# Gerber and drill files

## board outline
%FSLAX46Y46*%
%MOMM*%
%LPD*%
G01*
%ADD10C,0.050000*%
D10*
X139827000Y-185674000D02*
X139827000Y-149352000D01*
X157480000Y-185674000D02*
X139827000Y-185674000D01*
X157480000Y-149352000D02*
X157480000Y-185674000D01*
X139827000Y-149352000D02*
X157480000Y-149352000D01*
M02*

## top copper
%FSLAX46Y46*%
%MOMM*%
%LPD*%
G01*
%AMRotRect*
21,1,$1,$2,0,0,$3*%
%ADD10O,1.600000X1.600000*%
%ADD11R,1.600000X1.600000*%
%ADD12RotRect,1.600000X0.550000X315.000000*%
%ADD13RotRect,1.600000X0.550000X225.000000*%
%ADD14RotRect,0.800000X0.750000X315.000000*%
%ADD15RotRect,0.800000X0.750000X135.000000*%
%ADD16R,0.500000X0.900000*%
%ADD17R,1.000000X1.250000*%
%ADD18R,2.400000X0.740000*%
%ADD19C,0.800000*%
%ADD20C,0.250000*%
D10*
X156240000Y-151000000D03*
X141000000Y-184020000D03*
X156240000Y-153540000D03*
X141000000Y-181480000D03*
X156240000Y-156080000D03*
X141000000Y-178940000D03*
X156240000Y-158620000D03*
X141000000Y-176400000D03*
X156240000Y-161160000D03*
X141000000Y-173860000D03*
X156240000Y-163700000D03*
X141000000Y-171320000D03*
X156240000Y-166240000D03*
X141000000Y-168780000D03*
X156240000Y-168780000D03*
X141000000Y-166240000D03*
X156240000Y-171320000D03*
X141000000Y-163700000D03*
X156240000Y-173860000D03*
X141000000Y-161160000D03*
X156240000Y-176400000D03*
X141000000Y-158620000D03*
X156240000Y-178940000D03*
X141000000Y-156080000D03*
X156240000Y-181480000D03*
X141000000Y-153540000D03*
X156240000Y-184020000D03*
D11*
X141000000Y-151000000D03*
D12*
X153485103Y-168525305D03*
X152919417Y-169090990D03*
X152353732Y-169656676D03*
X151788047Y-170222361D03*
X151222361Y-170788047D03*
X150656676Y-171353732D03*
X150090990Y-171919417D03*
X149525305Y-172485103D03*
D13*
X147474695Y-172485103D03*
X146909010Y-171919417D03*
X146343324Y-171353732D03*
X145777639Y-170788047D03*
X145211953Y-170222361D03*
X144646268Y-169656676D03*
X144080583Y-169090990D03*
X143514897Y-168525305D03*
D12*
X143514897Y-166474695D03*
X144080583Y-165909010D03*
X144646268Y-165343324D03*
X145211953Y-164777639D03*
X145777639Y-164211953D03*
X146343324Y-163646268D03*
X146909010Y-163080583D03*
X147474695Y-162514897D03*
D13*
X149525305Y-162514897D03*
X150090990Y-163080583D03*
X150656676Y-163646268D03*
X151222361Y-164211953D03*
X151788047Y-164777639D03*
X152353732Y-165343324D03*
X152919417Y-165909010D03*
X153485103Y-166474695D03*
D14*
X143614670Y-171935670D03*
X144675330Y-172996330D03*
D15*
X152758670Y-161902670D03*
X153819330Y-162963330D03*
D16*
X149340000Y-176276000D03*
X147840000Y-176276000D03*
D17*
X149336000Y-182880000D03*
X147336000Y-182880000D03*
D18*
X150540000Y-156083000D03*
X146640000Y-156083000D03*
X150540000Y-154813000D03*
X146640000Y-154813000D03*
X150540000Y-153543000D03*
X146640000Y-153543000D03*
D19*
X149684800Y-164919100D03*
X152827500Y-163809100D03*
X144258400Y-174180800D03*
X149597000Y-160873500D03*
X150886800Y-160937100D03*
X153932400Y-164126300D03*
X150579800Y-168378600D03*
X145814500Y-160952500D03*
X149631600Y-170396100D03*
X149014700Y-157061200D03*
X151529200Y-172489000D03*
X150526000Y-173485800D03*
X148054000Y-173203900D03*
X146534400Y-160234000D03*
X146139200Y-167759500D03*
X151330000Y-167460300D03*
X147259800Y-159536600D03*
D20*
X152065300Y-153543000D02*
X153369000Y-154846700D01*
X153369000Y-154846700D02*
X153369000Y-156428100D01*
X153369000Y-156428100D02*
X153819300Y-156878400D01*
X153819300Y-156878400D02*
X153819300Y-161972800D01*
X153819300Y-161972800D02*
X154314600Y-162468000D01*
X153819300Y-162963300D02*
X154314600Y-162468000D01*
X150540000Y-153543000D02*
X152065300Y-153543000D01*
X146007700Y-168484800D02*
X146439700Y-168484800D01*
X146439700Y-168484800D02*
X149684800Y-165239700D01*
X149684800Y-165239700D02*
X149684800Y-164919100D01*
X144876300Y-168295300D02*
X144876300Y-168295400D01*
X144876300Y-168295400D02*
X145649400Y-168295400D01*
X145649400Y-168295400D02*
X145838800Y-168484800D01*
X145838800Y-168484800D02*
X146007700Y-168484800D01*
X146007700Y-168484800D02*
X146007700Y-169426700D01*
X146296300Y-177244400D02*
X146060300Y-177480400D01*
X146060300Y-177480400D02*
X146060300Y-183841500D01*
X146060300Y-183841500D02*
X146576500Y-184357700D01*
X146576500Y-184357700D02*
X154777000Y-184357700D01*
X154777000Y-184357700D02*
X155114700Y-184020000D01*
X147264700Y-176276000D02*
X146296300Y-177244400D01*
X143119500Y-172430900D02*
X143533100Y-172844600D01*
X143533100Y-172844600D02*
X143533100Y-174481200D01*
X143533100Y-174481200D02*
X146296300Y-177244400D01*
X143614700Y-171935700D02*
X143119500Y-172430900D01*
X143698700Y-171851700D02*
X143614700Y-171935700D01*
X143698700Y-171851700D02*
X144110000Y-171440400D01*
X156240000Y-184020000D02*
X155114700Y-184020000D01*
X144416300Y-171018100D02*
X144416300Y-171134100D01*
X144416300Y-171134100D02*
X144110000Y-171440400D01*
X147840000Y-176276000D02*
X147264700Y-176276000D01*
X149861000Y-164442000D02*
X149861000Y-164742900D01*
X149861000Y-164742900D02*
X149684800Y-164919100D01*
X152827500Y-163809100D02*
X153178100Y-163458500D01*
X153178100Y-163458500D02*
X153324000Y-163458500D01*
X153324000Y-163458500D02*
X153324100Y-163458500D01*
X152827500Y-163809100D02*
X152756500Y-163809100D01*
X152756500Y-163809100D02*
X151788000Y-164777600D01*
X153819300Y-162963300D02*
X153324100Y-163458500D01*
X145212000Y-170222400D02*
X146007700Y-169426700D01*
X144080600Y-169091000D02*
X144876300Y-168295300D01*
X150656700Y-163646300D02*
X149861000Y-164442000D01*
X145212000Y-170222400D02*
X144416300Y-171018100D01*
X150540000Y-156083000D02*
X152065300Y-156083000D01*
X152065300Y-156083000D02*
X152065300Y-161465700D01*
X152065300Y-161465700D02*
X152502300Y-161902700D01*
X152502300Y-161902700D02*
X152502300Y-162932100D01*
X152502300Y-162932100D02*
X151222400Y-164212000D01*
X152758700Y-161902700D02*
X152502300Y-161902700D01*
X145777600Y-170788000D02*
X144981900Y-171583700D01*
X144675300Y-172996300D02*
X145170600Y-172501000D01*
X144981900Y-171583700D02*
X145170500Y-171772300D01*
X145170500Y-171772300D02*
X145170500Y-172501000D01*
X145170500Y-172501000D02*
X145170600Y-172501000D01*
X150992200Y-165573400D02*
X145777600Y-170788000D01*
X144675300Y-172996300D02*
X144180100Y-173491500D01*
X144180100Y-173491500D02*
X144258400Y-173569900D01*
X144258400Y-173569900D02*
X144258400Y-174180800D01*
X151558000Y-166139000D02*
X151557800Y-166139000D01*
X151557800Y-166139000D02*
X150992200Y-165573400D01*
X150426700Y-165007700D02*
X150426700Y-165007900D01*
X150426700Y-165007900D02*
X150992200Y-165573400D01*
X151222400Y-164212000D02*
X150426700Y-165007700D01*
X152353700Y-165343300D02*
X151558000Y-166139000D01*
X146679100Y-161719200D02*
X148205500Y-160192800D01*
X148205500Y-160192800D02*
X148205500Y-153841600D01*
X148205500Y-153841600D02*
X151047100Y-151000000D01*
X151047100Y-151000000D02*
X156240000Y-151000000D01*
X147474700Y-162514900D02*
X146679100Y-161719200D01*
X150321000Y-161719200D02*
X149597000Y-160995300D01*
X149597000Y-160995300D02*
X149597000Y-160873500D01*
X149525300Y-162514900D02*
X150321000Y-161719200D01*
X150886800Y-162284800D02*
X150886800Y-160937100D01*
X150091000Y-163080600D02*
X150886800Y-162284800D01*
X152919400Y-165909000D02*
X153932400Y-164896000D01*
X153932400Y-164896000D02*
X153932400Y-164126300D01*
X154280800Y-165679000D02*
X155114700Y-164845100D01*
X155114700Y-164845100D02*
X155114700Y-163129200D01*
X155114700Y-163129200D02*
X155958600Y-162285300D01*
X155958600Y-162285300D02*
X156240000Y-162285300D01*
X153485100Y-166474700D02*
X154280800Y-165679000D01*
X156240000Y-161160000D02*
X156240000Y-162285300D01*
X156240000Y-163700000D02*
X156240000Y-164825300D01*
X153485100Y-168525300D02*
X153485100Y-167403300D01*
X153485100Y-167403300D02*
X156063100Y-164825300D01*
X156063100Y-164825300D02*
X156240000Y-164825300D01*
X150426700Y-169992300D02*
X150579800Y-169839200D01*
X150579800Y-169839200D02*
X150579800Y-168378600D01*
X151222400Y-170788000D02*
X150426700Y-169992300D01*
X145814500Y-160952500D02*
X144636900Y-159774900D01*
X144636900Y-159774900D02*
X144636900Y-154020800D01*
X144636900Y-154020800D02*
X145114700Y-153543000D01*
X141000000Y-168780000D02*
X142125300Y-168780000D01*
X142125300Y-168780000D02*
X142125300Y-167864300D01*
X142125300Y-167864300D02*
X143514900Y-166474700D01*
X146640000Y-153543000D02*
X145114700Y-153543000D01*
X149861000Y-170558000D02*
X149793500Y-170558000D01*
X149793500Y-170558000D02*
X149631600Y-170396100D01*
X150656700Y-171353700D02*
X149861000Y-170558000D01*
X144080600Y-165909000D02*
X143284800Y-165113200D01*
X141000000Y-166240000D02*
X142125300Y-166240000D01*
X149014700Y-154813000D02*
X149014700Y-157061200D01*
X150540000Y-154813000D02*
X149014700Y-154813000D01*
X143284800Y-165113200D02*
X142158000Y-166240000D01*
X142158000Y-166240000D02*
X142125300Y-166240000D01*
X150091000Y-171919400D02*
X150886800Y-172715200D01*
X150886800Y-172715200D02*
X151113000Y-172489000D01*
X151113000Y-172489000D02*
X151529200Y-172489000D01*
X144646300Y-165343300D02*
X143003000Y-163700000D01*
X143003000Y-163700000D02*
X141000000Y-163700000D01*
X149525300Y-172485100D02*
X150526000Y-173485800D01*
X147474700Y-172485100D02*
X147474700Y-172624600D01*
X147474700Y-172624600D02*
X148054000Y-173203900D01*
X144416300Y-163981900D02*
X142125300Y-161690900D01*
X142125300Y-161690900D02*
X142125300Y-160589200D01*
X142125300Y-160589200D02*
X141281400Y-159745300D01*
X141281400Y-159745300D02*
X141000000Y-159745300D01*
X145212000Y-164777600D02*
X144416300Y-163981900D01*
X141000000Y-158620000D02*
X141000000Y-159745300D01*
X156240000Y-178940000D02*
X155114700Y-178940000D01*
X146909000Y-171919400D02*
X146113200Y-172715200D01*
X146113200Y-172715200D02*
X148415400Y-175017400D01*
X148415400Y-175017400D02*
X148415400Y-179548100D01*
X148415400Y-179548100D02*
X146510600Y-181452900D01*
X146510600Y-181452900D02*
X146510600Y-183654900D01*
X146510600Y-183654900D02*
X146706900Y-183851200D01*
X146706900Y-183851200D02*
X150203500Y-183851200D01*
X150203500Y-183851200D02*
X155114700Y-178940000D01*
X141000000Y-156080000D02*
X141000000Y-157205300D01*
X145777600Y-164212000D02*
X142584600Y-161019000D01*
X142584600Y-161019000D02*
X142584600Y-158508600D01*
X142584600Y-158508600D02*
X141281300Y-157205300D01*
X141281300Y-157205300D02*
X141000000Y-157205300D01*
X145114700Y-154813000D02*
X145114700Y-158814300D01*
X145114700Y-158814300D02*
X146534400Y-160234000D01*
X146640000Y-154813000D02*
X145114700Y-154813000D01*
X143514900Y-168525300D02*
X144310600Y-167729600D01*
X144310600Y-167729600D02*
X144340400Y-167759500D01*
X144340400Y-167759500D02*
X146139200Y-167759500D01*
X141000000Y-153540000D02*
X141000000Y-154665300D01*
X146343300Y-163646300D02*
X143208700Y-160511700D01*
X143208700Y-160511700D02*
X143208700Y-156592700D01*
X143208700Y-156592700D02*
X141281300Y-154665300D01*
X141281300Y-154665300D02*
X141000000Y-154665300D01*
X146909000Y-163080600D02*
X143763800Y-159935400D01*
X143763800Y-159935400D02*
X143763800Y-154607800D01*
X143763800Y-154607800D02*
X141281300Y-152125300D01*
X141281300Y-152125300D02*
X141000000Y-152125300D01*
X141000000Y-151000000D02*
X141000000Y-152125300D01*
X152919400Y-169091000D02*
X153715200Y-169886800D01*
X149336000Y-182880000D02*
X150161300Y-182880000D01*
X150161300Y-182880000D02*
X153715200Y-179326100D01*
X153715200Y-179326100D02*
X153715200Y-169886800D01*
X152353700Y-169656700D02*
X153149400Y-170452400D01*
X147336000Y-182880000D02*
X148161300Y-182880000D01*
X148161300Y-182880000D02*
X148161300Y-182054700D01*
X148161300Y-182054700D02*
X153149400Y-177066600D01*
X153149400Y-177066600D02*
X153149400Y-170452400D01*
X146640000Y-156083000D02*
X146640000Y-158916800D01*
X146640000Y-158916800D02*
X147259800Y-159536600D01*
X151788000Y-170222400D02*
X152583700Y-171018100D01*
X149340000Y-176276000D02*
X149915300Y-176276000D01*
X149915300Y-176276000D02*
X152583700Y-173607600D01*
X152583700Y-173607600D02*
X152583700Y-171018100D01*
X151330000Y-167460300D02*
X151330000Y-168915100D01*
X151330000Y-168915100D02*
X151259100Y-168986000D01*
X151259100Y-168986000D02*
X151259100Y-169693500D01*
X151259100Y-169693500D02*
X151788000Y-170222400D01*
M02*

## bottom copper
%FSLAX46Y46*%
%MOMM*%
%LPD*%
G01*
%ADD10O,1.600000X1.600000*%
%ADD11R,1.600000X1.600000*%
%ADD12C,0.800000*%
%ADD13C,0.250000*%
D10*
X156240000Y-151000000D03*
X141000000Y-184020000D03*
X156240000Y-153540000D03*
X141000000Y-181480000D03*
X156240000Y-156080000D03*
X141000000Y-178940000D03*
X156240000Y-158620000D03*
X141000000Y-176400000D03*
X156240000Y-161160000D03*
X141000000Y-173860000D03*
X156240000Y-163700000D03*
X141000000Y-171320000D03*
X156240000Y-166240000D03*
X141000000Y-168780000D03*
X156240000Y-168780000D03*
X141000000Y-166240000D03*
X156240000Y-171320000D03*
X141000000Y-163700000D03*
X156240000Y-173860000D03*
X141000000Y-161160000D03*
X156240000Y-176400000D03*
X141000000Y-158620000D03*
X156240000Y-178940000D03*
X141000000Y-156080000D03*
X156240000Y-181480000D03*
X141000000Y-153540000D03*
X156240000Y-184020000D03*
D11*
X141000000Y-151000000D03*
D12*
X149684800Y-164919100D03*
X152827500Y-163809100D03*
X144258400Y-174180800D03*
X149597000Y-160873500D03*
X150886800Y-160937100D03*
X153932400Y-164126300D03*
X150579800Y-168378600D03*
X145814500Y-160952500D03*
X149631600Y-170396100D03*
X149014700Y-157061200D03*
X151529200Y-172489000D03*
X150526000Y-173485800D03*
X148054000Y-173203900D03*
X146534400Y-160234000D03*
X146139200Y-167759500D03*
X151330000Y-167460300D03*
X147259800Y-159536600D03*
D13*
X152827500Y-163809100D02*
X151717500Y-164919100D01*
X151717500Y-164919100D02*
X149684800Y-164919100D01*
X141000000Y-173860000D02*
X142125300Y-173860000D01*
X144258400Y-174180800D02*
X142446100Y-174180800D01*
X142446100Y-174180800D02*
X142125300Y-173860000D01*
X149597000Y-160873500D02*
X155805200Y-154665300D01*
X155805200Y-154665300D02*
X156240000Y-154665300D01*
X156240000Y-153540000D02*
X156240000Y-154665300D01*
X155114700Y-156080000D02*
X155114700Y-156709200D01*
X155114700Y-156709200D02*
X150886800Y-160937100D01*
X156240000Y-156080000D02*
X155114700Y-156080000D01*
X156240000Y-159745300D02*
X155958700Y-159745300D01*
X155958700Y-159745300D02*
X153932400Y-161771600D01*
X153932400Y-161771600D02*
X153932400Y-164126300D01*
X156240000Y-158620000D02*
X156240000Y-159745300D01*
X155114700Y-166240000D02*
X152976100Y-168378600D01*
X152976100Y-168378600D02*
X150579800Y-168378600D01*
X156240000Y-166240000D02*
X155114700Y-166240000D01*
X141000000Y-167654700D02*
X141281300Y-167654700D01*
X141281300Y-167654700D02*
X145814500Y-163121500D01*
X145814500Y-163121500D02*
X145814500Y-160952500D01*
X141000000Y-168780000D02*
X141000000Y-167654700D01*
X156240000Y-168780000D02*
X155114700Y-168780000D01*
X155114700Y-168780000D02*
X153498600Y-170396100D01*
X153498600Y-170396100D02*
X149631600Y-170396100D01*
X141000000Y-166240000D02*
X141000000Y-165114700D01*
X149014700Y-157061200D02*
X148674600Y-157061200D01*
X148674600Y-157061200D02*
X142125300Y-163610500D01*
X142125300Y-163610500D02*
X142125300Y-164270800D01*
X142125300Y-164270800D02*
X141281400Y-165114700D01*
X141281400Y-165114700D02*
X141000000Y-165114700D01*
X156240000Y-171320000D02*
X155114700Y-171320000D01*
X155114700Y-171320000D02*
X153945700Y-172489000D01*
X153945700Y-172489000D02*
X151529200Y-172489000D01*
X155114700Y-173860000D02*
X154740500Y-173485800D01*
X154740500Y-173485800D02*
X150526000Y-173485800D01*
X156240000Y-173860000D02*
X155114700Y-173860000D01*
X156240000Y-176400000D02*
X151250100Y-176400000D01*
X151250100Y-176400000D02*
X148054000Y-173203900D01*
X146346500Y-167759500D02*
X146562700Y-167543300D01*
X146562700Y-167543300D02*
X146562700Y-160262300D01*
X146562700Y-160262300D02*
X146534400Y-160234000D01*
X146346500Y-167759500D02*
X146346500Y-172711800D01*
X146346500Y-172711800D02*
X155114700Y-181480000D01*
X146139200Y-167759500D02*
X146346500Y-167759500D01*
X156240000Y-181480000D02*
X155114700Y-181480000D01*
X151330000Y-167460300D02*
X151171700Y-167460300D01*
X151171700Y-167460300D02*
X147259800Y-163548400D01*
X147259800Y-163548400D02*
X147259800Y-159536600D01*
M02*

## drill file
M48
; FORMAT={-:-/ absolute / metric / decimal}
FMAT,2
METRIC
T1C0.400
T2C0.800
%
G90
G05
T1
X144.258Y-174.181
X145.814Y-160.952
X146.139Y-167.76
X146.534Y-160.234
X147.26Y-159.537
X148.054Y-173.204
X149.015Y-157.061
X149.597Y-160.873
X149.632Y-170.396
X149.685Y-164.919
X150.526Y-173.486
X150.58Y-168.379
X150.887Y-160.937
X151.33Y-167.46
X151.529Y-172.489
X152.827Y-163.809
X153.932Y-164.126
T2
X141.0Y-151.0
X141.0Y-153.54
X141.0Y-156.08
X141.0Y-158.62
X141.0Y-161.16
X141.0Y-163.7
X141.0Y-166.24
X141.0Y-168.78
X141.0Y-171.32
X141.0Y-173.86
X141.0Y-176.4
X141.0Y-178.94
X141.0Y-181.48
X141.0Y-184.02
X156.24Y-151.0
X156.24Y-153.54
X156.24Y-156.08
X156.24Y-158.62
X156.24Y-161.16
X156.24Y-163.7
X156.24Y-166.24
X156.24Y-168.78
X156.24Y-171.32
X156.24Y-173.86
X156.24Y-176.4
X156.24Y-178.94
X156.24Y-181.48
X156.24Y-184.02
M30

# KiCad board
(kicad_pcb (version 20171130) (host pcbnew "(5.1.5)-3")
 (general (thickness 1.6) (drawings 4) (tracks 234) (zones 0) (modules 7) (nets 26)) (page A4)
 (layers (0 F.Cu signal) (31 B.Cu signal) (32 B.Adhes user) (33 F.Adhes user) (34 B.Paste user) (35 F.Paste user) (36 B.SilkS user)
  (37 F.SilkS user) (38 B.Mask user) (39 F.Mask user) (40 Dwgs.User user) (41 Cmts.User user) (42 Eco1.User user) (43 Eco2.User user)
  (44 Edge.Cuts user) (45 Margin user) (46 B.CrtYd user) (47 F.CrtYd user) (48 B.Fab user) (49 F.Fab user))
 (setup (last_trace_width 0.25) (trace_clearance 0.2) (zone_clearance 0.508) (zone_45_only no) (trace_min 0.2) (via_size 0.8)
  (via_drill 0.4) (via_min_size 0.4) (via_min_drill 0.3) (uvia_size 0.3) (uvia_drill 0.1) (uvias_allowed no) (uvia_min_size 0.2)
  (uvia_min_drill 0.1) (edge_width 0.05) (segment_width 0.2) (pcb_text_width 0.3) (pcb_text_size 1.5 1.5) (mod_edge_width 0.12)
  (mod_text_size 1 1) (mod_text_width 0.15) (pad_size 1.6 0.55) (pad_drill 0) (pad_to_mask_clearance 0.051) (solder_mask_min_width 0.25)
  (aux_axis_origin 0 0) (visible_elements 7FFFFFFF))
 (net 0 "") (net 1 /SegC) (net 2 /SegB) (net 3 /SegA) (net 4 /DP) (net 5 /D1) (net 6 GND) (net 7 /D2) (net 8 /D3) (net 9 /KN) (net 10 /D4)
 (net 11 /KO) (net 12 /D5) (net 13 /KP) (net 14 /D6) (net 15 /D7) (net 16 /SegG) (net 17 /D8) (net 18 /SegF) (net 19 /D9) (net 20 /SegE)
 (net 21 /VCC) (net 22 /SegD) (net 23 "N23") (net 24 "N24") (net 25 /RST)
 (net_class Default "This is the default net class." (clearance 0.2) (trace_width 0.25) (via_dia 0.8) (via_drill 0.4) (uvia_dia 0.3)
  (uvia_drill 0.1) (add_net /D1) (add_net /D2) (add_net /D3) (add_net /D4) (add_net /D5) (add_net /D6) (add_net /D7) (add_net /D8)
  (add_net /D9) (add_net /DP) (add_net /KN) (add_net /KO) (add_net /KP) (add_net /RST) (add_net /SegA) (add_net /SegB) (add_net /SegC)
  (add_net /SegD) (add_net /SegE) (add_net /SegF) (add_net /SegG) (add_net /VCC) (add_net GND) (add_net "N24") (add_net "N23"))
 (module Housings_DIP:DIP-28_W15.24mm (layer F.Cu) (at 141 151)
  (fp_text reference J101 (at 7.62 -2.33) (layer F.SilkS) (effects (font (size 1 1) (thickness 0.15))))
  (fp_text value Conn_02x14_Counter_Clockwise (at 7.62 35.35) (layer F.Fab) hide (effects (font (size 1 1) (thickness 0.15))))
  (pad 28 thru_hole oval (at 15.24 0) (size 1.6 1.6) (drill 0.8) (layers *.Cu *.Mask) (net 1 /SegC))
  (pad 14 thru_hole oval (at 0 33.02) (size 1.6 1.6) (drill 0.8) (layers *.Cu *.Mask))
  (pad 27 thru_hole oval (at 15.24 2.54) (size 1.6 1.6) (drill 0.8) (layers *.Cu *.Mask) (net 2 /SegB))
  (pad 13 thru_hole oval (at 0 30.48) (size 1.6 1.6) (drill 0.8) (layers *.Cu *.Mask))
  (pad 26 thru_hole oval (at 15.24 5.08) (size 1.6 1.6) (drill 0.8) (layers *.Cu *.Mask) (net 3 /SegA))
  (pad 12 thru_hole oval (at 0 27.94) (size 1.6 1.6) (drill 0.8) (layers *.Cu *.Mask))
  (pad 25 thru_hole oval (at 15.24 7.62) (size 1.6 1.6) (drill 0.8) (layers *.Cu *.Mask) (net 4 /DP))
  (pad 11 thru_hole oval (at 0 25.4) (size 1.6 1.6) (drill 0.8) (layers *.Cu *.Mask))
  (pad 24 thru_hole oval (at 15.24 10.16) (size 1.6 1.6) (drill 0.8) (layers *.Cu *.Mask) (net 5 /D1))
  (pad 10 thru_hole oval (at 0 22.86) (size 1.6 1.6) (drill 0.8) (layers *.Cu *.Mask) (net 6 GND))
  (pad 23 thru_hole oval (at 15.24 12.7) (size 1.6 1.6) (drill 0.8) (layers *.Cu *.Mask) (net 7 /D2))
  (pad 9 thru_hole oval (at 0 20.32) (size 1.6 1.6) (drill 0.8) (layers *.Cu *.Mask))
  (pad 22 thru_hole oval (at 15.24 15.24) (size 1.6 1.6) (drill 0.8) (layers *.Cu *.Mask) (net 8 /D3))
  (pad 8 thru_hole oval (at 0 17.78) (size 1.6 1.6) (drill 0.8) (layers *.Cu *.Mask) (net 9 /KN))
  (pad 21 thru_hole oval (at 15.24 17.78) (size 1.6 1.6) (drill 0.8) (layers *.Cu *.Mask) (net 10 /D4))
  (pad 7 thru_hole oval (at 0 15.24) (size 1.6 1.6) (drill 0.8) (layers *.Cu *.Mask) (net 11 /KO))
  (pad 20 thru_hole oval (at 15.24 20.32) (size 1.6 1.6) (drill 0.8) (layers *.Cu *.Mask) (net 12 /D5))
  (pad 6 thru_hole oval (at 0 12.7) (size 1.6 1.6) (drill 0.8) (layers *.Cu *.Mask) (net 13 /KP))
  (pad 19 thru_hole oval (at 15.24 22.86) (size 1.6 1.6) (drill 0.8) (layers *.Cu *.Mask) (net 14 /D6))
  (pad 5 thru_hole oval (at 0 10.16) (size 1.6 1.6) (drill 0.8) (layers *.Cu *.Mask))
  (pad 18 thru_hole oval (at 15.24 25.4) (size 1.6 1.6) (drill 0.8) (layers *.Cu *.Mask) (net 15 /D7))
  (pad 4 thru_hole oval (at 0 7.62) (size 1.6 1.6) (drill 0.8) (layers *.Cu *.Mask) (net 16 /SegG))
  (pad 17 thru_hole oval (at 15.24 27.94) (size 1.6 1.6) (drill 0.8) (layers *.Cu *.Mask) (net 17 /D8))
  (pad 3 thru_hole oval (at 0 5.08) (size 1.6 1.6) (drill 0.8) (layers *.Cu *.Mask) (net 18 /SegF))
  (pad 16 thru_hole oval (at 15.24 30.48) (size 1.6 1.6) (drill 0.8) (layers *.Cu *.Mask) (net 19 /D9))
  (pad 2 thru_hole oval (at 0 2.54) (size 1.6 1.6) (drill 0.8) (layers *.Cu *.Mask) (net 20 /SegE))
  (pad 15 thru_hole oval (at 15.24 33.02) (size 1.6 1.6) (drill 0.8) (layers *.Cu *.Mask) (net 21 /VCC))
  (pad 1 thru_hole rect (at 0 0) (size 1.6 1.6) (drill 0.8) (layers *.Cu *.Mask) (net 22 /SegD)))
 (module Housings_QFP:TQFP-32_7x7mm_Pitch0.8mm (layer F.Cu) (at 148.5 167.5 225)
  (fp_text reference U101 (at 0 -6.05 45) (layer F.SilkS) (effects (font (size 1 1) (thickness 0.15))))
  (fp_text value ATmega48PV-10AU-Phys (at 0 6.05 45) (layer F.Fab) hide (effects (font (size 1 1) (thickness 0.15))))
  (pad 32 smd rect (at -2.8 -4.25 315) (size 1.6 0.55) (layers F.Cu F.Paste F.Mask) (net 7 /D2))
  (pad 31 smd rect (at -2 -4.25 315) (size 1.6 0.55) (layers F.Cu F.Paste F.Mask) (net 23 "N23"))
  (pad 30 smd rect (at -1.2 -4.25 315) (size 1.6 0.55) (layers F.Cu F.Paste F.Mask) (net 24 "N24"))
  (pad 29 smd rect (at -0.4 -4.25 315) (size 1.6 0.55) (layers F.Cu F.Paste F.Mask) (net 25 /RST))
  (pad 28 smd rect (at 0.4 -4.25 315) (size 1.6 0.55) (layers F.Cu F.Paste F.Mask) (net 8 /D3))
  (pad 27 smd rect (at 1.2 -4.25 315) (size 1.6 0.55) (layers F.Cu F.Paste F.Mask) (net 10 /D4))
  (pad 26 smd rect (at 2 -4.25 315) (size 1.6 0.55) (layers F.Cu F.Paste F.Mask) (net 12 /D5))
  (pad 25 smd rect (at 2.8 -4.25 315) (size 1.6 0.55) (layers F.Cu F.Paste F.Mask) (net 14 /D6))
  (pad 24 smd rect (at 4.25 -2.8 225) (size 1.6 0.55) (layers F.Cu F.Paste F.Mask) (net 15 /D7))
  (pad 23 smd rect (at 4.25 -2 225) (size 1.6 0.55) (layers F.Cu F.Paste F.Mask) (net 17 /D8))
  (pad 22 smd rect (at 4.25 -1.2 225) (size 1.6 0.55) (layers F.Cu F.Paste F.Mask))
  (pad 21 smd rect (at 4.25 -0.4 225) (size 1.6 0.55) (layers F.Cu F.Paste F.Mask) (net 6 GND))
  (pad 20 smd rect (at 4.25 0.4 225) (size 1.6 0.55) (layers F.Cu F.Paste F.Mask) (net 21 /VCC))
  (pad 19 smd rect (at 4.25 1.2 225) (size 1.6 0.55) (layers F.Cu F.Paste F.Mask))
  (pad 18 smd rect (at 4.25 2 225) (size 1.6 0.55) (layers F.Cu F.Paste F.Mask) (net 21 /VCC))
  (pad 17 smd rect (at 4.25 2.8 225) (size 1.6 0.55) (layers F.Cu F.Paste F.Mask) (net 19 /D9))
  (pad 16 smd rect (at 2.8 4.25 315) (size 1.6 0.55) (layers F.Cu F.Paste F.Mask) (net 9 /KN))
  (pad 15 smd rect (at 2 4.25 315) (size 1.6 0.55) (layers F.Cu F.Paste F.Mask) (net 11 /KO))
  (pad 14 smd rect (at 1.2 4.25 315) (size 1.6 0.55) (layers F.Cu F.Paste F.Mask) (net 13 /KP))
  (pad 13 smd rect (at 0.4 4.25 315) (size 1.6 0.55) (layers F.Cu F.Paste F.Mask) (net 16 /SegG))
  (pad 12 smd rect (at -0.4 4.25 315) (size 1.6 0.55) (layers F.Cu F.Paste F.Mask) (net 18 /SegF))
  (pad 11 smd rect (at -1.2 4.25 315) (size 1.6 0.55) (layers F.Cu F.Paste F.Mask) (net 20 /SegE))
  (pad 10 smd rect (at -2 4.25 315) (size 1.6 0.55) (layers F.Cu F.Paste F.Mask) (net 22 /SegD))
  (pad 9 smd rect (at -2.8 4.25 315) (size 1.6 0.55) (layers F.Cu F.Paste F.Mask) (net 1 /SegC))
  (pad 8 smd rect (at -4.25 2.8 225) (size 1.6 0.55) (layers F.Cu F.Paste F.Mask) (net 2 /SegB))
  (pad 7 smd rect (at -4.25 2 225) (size 1.6 0.55) (layers F.Cu F.Paste F.Mask) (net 3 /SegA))
  (pad 6 smd rect (at -4.25 1.2 225) (size 1.6 0.55) (layers F.Cu F.Paste F.Mask) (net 21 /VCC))
  (pad 5 smd rect (at -4.25 0.4 225) (size 1.6 0.55) (layers F.Cu F.Paste F.Mask) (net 6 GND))
  (pad 4 smd rect (at -4.25 -0.4 225) (size 1.6 0.55) (layers F.Cu F.Paste F.Mask) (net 21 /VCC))
  (pad 3 smd rect (at -4.25 -1.2 225) (size 1.6 0.55) (layers F.Cu F.Paste F.Mask) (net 6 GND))
  (pad 2 smd rect (at -4.25 -2 225) (size 1.6 0.55) (layers F.Cu F.Paste F.Mask) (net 4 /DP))
  (pad 1 smd rect (at -4.25 -2.8 225) (size 1.6 0.55) (layers F.Cu F.Paste F.Mask) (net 5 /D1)))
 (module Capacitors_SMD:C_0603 (layer F.Cu) (at 144.145 172.466 315)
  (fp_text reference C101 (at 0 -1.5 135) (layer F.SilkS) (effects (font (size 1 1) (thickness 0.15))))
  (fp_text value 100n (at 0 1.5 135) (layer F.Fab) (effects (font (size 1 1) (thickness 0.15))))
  (pad 1 smd rect (at -0.75 0 315) (size 0.8 0.75) (layers F.Cu F.Paste F.Mask) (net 21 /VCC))
  (pad 2 smd rect (at 0.75 0 315) (size 0.8 0.75) (layers F.Cu F.Paste F.Mask) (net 6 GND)))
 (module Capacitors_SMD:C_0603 (layer F.Cu) (at 153.289 162.433 135)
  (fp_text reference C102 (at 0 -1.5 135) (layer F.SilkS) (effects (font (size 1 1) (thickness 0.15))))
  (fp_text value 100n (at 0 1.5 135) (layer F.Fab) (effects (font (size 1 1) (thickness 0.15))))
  (pad 2 smd rect (at 0.75 0 135) (size 0.8 0.75) (layers F.Cu F.Paste F.Mask) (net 6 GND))
  (pad 1 smd rect (at -0.75 0 135) (size 0.8 0.75) (layers F.Cu F.Paste F.Mask) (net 21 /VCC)))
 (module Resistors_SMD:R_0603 (layer F.Cu) (at 148.59 176.276)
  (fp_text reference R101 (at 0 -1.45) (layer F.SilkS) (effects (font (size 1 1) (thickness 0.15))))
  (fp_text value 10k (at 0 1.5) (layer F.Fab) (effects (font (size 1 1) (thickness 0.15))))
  (pad 2 smd rect (at 0.75 0) (size 0.5 0.9) (layers F.Cu F.Paste F.Mask) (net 25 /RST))
  (pad 1 smd rect (at -0.75 0) (size 0.5 0.9) (layers F.Cu F.Paste F.Mask) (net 21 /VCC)))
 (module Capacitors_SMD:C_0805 (layer F.Cu) (at 148.336 182.88)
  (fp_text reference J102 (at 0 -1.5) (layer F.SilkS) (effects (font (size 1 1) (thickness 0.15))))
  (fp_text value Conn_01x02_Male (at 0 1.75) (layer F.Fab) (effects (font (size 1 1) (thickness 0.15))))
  (pad 2 smd rect (at 1 0) (size 1 1.25) (layers F.Cu F.Paste F.Mask) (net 23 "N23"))
  (pad 1 smd rect (at -1 0) (size 1 1.25) (layers F.Cu F.Paste F.Mask) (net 24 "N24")))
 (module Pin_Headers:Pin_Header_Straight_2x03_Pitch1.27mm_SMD (layer F.Cu) (at 148.59 154.813)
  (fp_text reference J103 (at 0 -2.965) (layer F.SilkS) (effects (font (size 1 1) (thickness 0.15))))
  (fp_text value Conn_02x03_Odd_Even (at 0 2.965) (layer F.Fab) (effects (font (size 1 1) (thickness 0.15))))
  (pad 6 smd rect (at 1.95 1.27) (size 2.4 0.74) (layers F.Cu F.Paste F.Mask) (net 6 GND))
  (pad 5 smd rect (at -1.95 1.27) (size 2.4 0.74) (layers F.Cu F.Paste F.Mask) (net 25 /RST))
  (pad 4 smd rect (at 1.95 0) (size 2.4 0.74) (layers F.Cu F.Paste F.Mask) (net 11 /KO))
  (pad 3 smd rect (at -1.95 0) (size 2.4 0.74) (layers F.Cu F.Paste F.Mask) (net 19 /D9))
  (pad 2 smd rect (at 1.95 -1.27) (size 2.4 0.74) (layers F.Cu F.Paste F.Mask) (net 21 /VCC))
  (pad 1 smd rect (at -1.95 -1.27) (size 2.4 0.74) (layers F.Cu F.Paste F.Mask) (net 9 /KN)))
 (gr_line (start 139.827 185.674) (end 139.827 149.352) (layer Edge.Cuts) (width 0.05))
 (gr_line (start 157.48 185.674) (end 139.827 185.674) (layer Edge.Cuts) (width 0.05))
 (gr_line (start 157.48 149.352) (end 157.48 185.674) (layer Edge.Cuts) (width 0.05))
 (gr_line (start 139.827 149.352) (end 157.48 149.352) (layer Edge.Cuts) (width 0.05))
 (segment (start 152.0653 153.543) (end 153.369 154.8467) (width 0.25) (layer F.Cu) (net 21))
 (segment (start 153.369 154.8467) (end 153.369 156.4281) (width 0.25) (layer F.Cu) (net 21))
 (segment (start 153.369 156.4281) (end 153.8193 156.8784) (width 0.25) (layer F.Cu) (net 21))
 (segment (start 153.8193 156.8784) (end 153.8193 161.9728) (width 0.25) (layer F.Cu) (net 21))
 (segment (start 153.8193 161.9728) (end 154.3146 162.468) (width 0.25) (layer F.Cu) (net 21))
 (segment (start 153.8193 162.9633) (end 154.3146 162.468) (width 0.25) (layer F.Cu) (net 21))
 (segment (start 150.54 153.543) (end 152.0653 153.543) (width 0.25) (layer F.Cu) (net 21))
 (segment (start 146.0077 168.4848) (end 146.4397 168.4848) (width 0.25) (layer F.Cu) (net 21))
 (segment (start 146.4397 168.4848) (end 149.6848 165.2397) (width 0.25) (layer F.Cu) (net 21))
 (segment (start 149.6848 165.2397) (end 149.6848 164.9191) (width 0.25) (layer F.Cu) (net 21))
 (segment (start 144.8763 168.2953) (end 144.8763 168.2954) (width 0.25) (layer F.Cu) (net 21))
 (segment (start 144.8763 168.2954) (end 145.6494 168.2954) (width 0.25) (layer F.Cu) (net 21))
 (segment (start 145.6494 168.2954) (end 145.8388 168.4848) (width 0.25) (layer F.Cu) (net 21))
 (segment (start 145.8388 168.4848) (end 146.0077 168.4848) (width 0.25) (layer F.Cu) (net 21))
 (segment (start 146.0077 168.4848) (end 146.0077 169.4267) (width 0.25) (layer F.Cu) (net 21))
 (segment (start 146.2963 177.2444) (end 146.0603 177.4804) (width 0.25) (layer F.Cu) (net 21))
 (segment (start 146.0603 177.4804) (end 146.0603 183.8415) (width 0.25) (layer F.Cu) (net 21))
 (segment (start 146.0603 183.8415) (end 146.5765 184.3577) (width 0.25) (layer F.Cu) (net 21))
 (segment (start 146.5765 184.3577) (end 154.777 184.3577) (width 0.25) (layer F.Cu) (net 21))
 (segment (start 154.777 184.3577) (end 155.1147 184.02) (width 0.25) (layer F.Cu) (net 21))
 (segment (start 147.2647 176.276) (end 146.2963 177.2444) (width 0.25) (layer F.Cu) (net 21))
 (segment (start 143.1195 172.4309) (end 143.5331 172.8446) (width 0.25) (layer F.Cu) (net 21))
 (segment (start 143.5331 172.8446) (end 143.5331 174.4812) (width 0.25) (layer F.Cu) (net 21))
 (segment (start 143.5331 174.4812) (end 146.2963 177.2444) (width 0.25) (layer F.Cu) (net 21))
 (segment (start 143.6147 171.9357) (end 143.1195 172.4309) (width 0.25) (layer F.Cu) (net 21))
 (segment (start 143.6987 171.8517) (end 143.6147 171.9357) (width 0.25) (layer F.Cu) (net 21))
 (segment (start 143.6987 171.8517) (end 144.11 171.4404) (width 0.25) (layer F.Cu) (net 21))
 (segment (start 156.24 184.02) (end 155.1147 184.02) (width 0.25) (layer F.Cu) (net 21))
 (segment (start 144.4163 171.0181) (end 144.4163 171.1341) (width 0.25) (layer F.Cu) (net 21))
 (segment (start 144.4163 171.1341) (end 144.11 171.4404) (width 0.25) (layer F.Cu) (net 21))
 (segment (start 147.84 176.276) (end 147.2647 176.276) (width 0.25) (layer F.Cu) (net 21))
 (segment (start 149.861 164.442) (end 149.861 164.7429) (width 0.25) (layer F.Cu) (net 21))
 (segment (start 149.861 164.7429) (end 149.6848 164.9191) (width 0.25) (layer F.Cu) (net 21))
 (segment (start 152.8275 163.8091) (end 151.7175 164.9191) (width 0.25) (layer B.Cu) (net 21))
 (segment (start 151.7175 164.9191) (end 149.6848 164.9191) (width 0.25) (layer B.Cu) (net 21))
 (segment (start 152.8275 163.8091) (end 153.1781 163.4585) (width 0.25) (layer F.Cu) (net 21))
 (segment (start 153.1781 163.4585) (end 153.324 163.4585) (width 0.25) (layer F.Cu) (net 21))
 (segment (start 153.324 163.4585) (end 153.3241 163.4585) (width 0.25) (layer F.Cu) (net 21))
 (segment (start 152.8275 163.8091) (end 152.7565 163.8091) (width 0.25) (layer F.Cu) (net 21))
 (segment (start 152.7565 163.8091) (end 151.788 164.7776) (width 0.25) (layer F.Cu) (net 21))
 (segment (start 153.8193 162.9633) (end 153.3241 163.4585) (width 0.25) (layer F.Cu) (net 21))
 (segment (start 145.212 170.2224) (end 146.0077 169.4267) (width 0.25) (layer F.Cu) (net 21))
 (segment (start 144.0806 169.091) (end 144.8763 168.2953) (width 0.25) (layer F.Cu) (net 21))
 (segment (start 150.6567 163.6463) (end 149.861 164.442) (width 0.25) (layer F.Cu) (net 21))
 (segment (start 145.212 170.2224) (end 144.4163 171.0181) (width 0.25) (layer F.Cu) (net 21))
 (via (at 149.6848 164.9191) (size 0.8) (layers F.Cu B.Cu) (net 21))
 (via (at 152.8275 163.8091) (size 0.8) (layers F.Cu B.Cu) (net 21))
 (segment (start 150.54 156.083) (end 152.0653 156.083) (width 0.25) (layer F.Cu) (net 6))
 (segment (start 152.0653 156.083) (end 152.0653 161.4657) (width 0.25) (layer F.Cu) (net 6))
 (segment (start 152.0653 161.4657) (end 152.5023 161.9027) (width 0.25) (layer F.Cu) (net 6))
 (segment (start 152.5023 161.9027) (end 152.5023 162.9321) (width 0.25) (layer F.Cu) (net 6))
 (segment (start 152.5023 162.9321) (end 151.2224 164.212) (width 0.25) (layer F.Cu) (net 6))
 (segment (start 152.7587 161.9027) (end 152.5023 161.9027) (width 0.25) (layer F.Cu) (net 6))
 (segment (start 145.7776 170.788) (end 144.9819 171.5837) (width 0.25) (layer F.Cu) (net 6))
 (segment (start 144.6753 172.9963) (end 145.1706 172.501) (width 0.25) (layer F.Cu) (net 6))
 (segment (start 144.9819 171.5837) (end 145.1705 171.7723) (width 0.25) (layer F.Cu) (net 6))
 (segment (start 145.1705 171.7723) (end 145.1705 172.501) (width 0.25) (layer F.Cu) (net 6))
 (segment (start 145.1705 172.501) (end 145.1706 172.501) (width 0.25) (layer F.Cu) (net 6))
 (segment (start 150.9922 165.5734) (end 145.7776 170.788) (width 0.25) (layer F.Cu) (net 6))
 (segment (start 141 173.86) (end 142.1253 173.86) (width 0.25) (layer B.Cu) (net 6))
 (segment (start 144.6753 172.9963) (end 144.1801 173.4915) (width 0.25) (layer F.Cu) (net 6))
 (segment (start 144.2584 174.1808) (end 142.4461 174.1808) (width 0.25) (layer B.Cu) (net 6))
 (segment (start 142.4461 174.1808) (end 142.1253 173.86) (width 0.25) (layer B.Cu) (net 6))
 (segment (start 144.1801 173.4915) (end 144.2584 173.5699) (width 0.25) (layer F.Cu) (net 6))
 (segment (start 144.2584 173.5699) (end 144.2584 174.1808) (width 0.25) (layer F.Cu) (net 6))
 (segment (start 151.558 166.139) (end 151.5578 166.139) (width 0.25) (layer F.Cu) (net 6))
 (segment (start 151.5578 166.139) (end 150.9922 165.5734) (width 0.25) (layer F.Cu) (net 6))
 (segment (start 150.4267 165.0077) (end 150.4267 165.0079) (width 0.25) (layer F.Cu) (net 6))
 (segment (start 150.4267 165.0079) (end 150.9922 165.5734) (width 0.25) (layer F.Cu) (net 6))
 (segment (start 151.2224 164.212) (end 150.4267 165.0077) (width 0.25) (layer F.Cu) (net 6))
 (segment (start 152.3537 165.3433) (end 151.558 166.139) (width 0.25) (layer F.Cu) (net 6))
 (via (at 144.2584 174.1808) (size 0.8) (layers F.Cu B.Cu) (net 6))
 (segment (start 146.6791 161.7192) (end 148.2055 160.1928) (width 0.25) (layer F.Cu) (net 1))
 (segment (start 148.2055 160.1928) (end 148.2055 153.8416) (width 0.25) (layer F.Cu) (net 1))
 (segment (start 148.2055 153.8416) (end 151.0471 151) (width 0.25) (layer F.Cu) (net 1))
 (segment (start 151.0471 151) (end 156.24 151) (width 0.25) (layer F.Cu) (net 1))
 (segment (start 147.4747 162.5149) (end 146.6791 161.7192) (width 0.25) (layer F.Cu) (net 1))
 (segment (start 150.321 161.7192) (end 149.597 160.9953) (width 0.25) (layer F.Cu) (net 2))
 (segment (start 149.597 160.9953) (end 149.597 160.8735) (width 0.25) (layer F.Cu) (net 2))
 (segment (start 149.597 160.8735) (end 155.8052 154.6653) (width 0.25) (layer B.Cu) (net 2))
 (segment (start 155.8052 154.6653) (end 156.24 154.6653) (width 0.25) (layer B.Cu) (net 2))
 (segment (start 156.24 153.54) (end 156.24 154.6653) (width 0.25) (layer B.Cu) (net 2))
 (segment (start 149.5253 162.5149) (end 150.321 161.7192) (width 0.25) (layer F.Cu) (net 2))
 (via (at 149.597 160.8735) (size 0.8) (layers F.Cu B.Cu) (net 2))
 (segment (start 150.8868 162.2848) (end 150.8868 160.9371) (width 0.25) (layer F.Cu) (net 3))
 (segment (start 155.1147 156.08) (end 155.1147 156.7092) (width 0.25) (layer B.Cu) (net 3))
 (segment (start 155.1147 156.7092) (end 150.8868 160.9371) (width 0.25) (layer B.Cu) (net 3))
 (segment (start 156.24 156.08) (end 155.1147 156.08) (width 0.25) (layer B.Cu) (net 3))
 (segment (start 150.091 163.0806) (end 150.8868 162.2848) (width 0.25) (layer F.Cu) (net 3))
 (via (at 150.8868 160.9371) (size 0.8) (layers F.Cu B.Cu) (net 3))
 (segment (start 152.9194 165.909) (end 153.9324 164.896) (width 0.25) (layer F.Cu) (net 4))
 (segment (start 153.9324 164.896) (end 153.9324 164.1263) (width 0.25) (layer F.Cu) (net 4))
 (segment (start 156.24 159.7453) (end 155.9587 159.7453) (width 0.25) (layer B.Cu) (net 4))
 (segment (start 155.9587 159.7453) (end 153.9324 161.7716) (width 0.25) (layer B.Cu) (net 4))
 (segment (start 153.9324 161.7716) (end 153.9324 164.1263) (width 0.25) (layer B.Cu) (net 4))
 (segment (start 156.24 158.62) (end 156.24 159.7453) (width 0.25) (layer B.Cu) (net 4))
 (via (at 153.9324 164.1263) (size 0.8) (layers F.Cu B.Cu) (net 4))
 (segment (start 154.2808 165.679) (end 155.1147 164.8451) (width 0.25) (layer F.Cu) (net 5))
 (segment (start 155.1147 164.8451) (end 155.1147 163.1292) (width 0.25) (layer F.Cu) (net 5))
 (segment (start 155.1147 163.1292) (end 155.9586 162.2853) (width 0.25) (layer F.Cu) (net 5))
 (segment (start 155.9586 162.2853) (end 156.24 162.2853) (width 0.25) (layer F.Cu) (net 5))
 (segment (start 153.4851 166.4747) (end 154.2808 165.679) (width 0.25) (layer F.Cu) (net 5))
 (segment (start 156.24 161.16) (end 156.24 162.2853) (width 0.25) (layer F.Cu) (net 5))
 (segment (start 156.24 163.7) (end 156.24 164.8253) (width 0.25) (layer F.Cu) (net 7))
 (segment (start 153.4851 168.5253) (end 153.4851 167.4033) (width 0.25) (layer F.Cu) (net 7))
 (segment (start 153.4851 167.4033) (end 156.0631 164.8253) (width 0.25) (layer F.Cu) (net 7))
 (segment (start 156.0631 164.8253) (end 156.24 164.8253) (width 0.25) (layer F.Cu) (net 7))
 (segment (start 150.4267 169.9923) (end 150.5798 169.8392) (width 0.25) (layer F.Cu) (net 8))
 (segment (start 150.5798 169.8392) (end 150.5798 168.3786) (width 0.25) (layer F.Cu) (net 8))
 (segment (start 155.1147 166.24) (end 152.9761 168.3786) (width 0.25) (layer B.Cu) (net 8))
 (segment (start 152.9761 168.3786) (end 150.5798 168.3786) (width 0.25) (layer B.Cu) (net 8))
 (segment (start 156.24 166.24) (end 155.1147 166.24) (width 0.25) (layer B.Cu) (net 8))
 (segment (start 151.2224 170.788) (end 150.4267 169.9923) (width 0.25) (layer F.Cu) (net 8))
 (via (at 150.5798 168.3786) (size 0.8) (layers F.Cu B.Cu) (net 8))
 (segment (start 145.8145 160.9525) (end 144.6369 159.7749) (width 0.25) (layer F.Cu) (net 9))
 (segment (start 144.6369 159.7749) (end 144.6369 154.0208) (width 0.25) (layer F.Cu) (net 9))
 (segment (start 144.6369 154.0208) (end 145.1147 153.543) (width 0.25) (layer F.Cu) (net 9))
 (segment (start 141 168.78) (end 142.1253 168.78) (width 0.25) (layer F.Cu) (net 9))
 (segment (start 142.1253 168.78) (end 142.1253 167.8643) (width 0.25) (layer F.Cu) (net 9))
 (segment (start 142.1253 167.8643) (end 143.5149 166.4747) (width 0.25) (layer F.Cu) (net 9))
 (segment (start 141 167.6547) (end 141.2813 167.6547) (width 0.25) (layer B.Cu) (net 9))
 (segment (start 141.2813 167.6547) (end 145.8145 163.1215) (width 0.25) (layer B.Cu) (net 9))
 (segment (start 145.8145 163.1215) (end 145.8145 160.9525) (width 0.25) (layer B.Cu) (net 9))
 (segment (start 146.64 153.543) (end 145.1147 153.543) (width 0.25) (layer F.Cu) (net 9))
 (segment (start 141 168.78) (end 141 167.6547) (width 0.25) (layer B.Cu) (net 9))
 (via (at 145.8145 160.9525) (size 0.8) (layers F.Cu B.Cu) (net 9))
 (segment (start 156.24 168.78) (end 155.1147 168.78) (width 0.25) (layer B.Cu) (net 10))
 (segment (start 149.861 170.558) (end 149.7935 170.558) (width 0.25) (layer F.Cu) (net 10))
 (segment (start 149.7935 170.558) (end 149.6316 170.3961) (width 0.25) (layer F.Cu) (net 10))
 (segment (start 155.1147 168.78) (end 153.4986 170.3961) (width 0.25) (layer B.Cu) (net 10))
 (segment (start 153.4986 170.3961) (end 149.6316 170.3961) (width 0.25) (layer B.Cu) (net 10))
 (segment (start 150.6567 171.3537) (end 149.861 170.558) (width 0.25) (layer F.Cu) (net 10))
 (via (at 149.6316 170.3961) (size 0.8) (layers F.Cu B.Cu) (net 10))
 (segment (start 141 166.24) (end 141 165.1147) (width 0.25) (layer B.Cu) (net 11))
 (segment (start 144.0806 165.909) (end 143.2848 165.1132) (width 0.25) (layer F.Cu) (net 11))
 (segment (start 141 166.24) (end 142.1253 166.24) (width 0.25) (layer F.Cu) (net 11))
 (segment (start 149.0147 157.0612) (end 148.6746 157.0612) (width 0.25) (layer B.Cu) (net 11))
 (segment (start 148.6746 157.0612) (end 142.1253 163.6105) (width 0.25) (layer B.Cu) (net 11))
 (segment (start 142.1253 163.6105) (end 142.1253 164.2708) (width 0.25) (layer B.Cu) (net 11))
 (segment (start 142.1253 164.2708) (end 141.2814 165.1147) (width 0.25) (layer B.Cu) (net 11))
 (segment (start 141.2814 165.1147) (end 141 165.1147) (width 0.25) (layer B.Cu) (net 11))
 (segment (start 149.0147 154.813) (end 149.0147 157.0612) (width 0.25) (layer F.Cu) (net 11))
 (segment (start 150.54 154.813) (end 149.0147 154.813) (width 0.25) (layer F.Cu) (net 11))
 (segment (start 143.2848 165.1132) (end 142.158 166.24) (width 0.25) (layer F.Cu) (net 11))
 (segment (start 142.158 166.24) (end 142.1253 166.24) (width 0.25) (layer F.Cu) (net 11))
 (via (at 149.0147 157.0612) (size 0.8) (layers F.Cu B.Cu) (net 11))
 (segment (start 150.091 171.9194) (end 150.8868 172.7152) (width 0.25) (layer F.Cu) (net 12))
 (segment (start 156.24 171.32) (end 155.1147 171.32) (width 0.25) (layer B.Cu) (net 12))
 (segment (start 150.8868 172.7152) (end 151.113 172.489) (width 0.25) (layer F.Cu) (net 12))
 (segment (start 151.113 172.489) (end 151.5292 172.489) (width 0.25) (layer F.Cu) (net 12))
 (segment (start 155.1147 171.32) (end 153.9457 172.489) (width 0.25) (layer B.Cu) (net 12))
 (segment (start 153.9457 172.489) (end 151.5292 172.489) (width 0.25) (layer B.Cu) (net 12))
 (via (at 151.5292 172.489) (size 0.8) (layers F.Cu B.Cu) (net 12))
 (segment (start 144.6463 165.3433) (end 143.003 163.7) (width 0.25) (layer F.Cu) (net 13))
 (segment (start 143.003 163.7) (end 141 163.7) (width 0.25) (layer F.Cu) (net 13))
 (segment (start 149.5253 172.4851) (end 150.526 173.4858) (width 0.25) (layer F.Cu) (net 14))
 (segment (start 155.1147 173.86) (end 154.7405 173.4858) (width 0.25) (layer B.Cu) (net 14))
 (segment (start 154.7405 173.4858) (end 150.526 173.4858) (width 0.25) (layer B.Cu) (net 14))
 (segment (start 156.24 173.86) (end 155.1147 173.86) (width 0.25) (layer B.Cu) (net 14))
 (via (at 150.526 173.4858) (size 0.8) (layers F.Cu B.Cu) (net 14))
 (segment (start 147.4747 172.4851) (end 147.4747 172.6246) (width 0.25) (layer F.Cu) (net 15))
 (segment (start 147.4747 172.6246) (end 148.054 173.2039) (width 0.25) (layer F.Cu) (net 15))
 (segment (start 156.24 176.4) (end 151.2501 176.4) (width 0.25) (layer B.Cu) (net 15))
 (segment (start 151.2501 176.4) (end 148.054 173.2039) (width 0.25) (layer B.Cu) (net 15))
 (via (at 148.054 173.2039) (size 0.8) (layers F.Cu B.Cu) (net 15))
 (segment (start 144.4163 163.9819) (end 142.1253 161.6909) (width 0.25) (layer F.Cu) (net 16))
 (segment (start 142.1253 161.6909) (end 142.1253 160.5892) (width 0.25) (layer F.Cu) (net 16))
 (segment (start 142.1253 160.5892) (end 141.2814 159.7453) (width 0.25) (layer F.Cu) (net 16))
 (segment (start 141.2814 159.7453) (end 141 159.7453) (width 0.25) (layer F.Cu) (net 16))
 (segment (start 145.212 164.7776) (end 144.4163 163.9819) (width 0.25) (layer F.Cu) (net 16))
 (segment (start 141 158.62) (end 141 159.7453) (width 0.25) (layer F.Cu) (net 16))
 (segment (start 156.24 178.94) (end 155.1147 178.94) (width 0.25) (layer F.Cu) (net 17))
 (segment (start 146.909 171.9194) (end 146.1132 172.7152) (width 0.25) (layer F.Cu) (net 17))
 (segment (start 146.1132 172.7152) (end 148.4154 175.0174) (width 0.25) (layer F.Cu) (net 17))
 (segment (start 148.4154 175.0174) (end 148.4154 179.5481) (width 0.25) (layer F.Cu) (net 17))
 (segment (start 148.4154 179.5481) (end 146.5106 181.4529) (width 0.25) (layer F.Cu) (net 17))
 (segment (start 146.5106 181.4529) (end 146.5106 183.6549) (width 0.25) (layer F.Cu) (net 17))
 (segment (start 146.5106 183.6549) (end 146.7069 183.8512) (width 0.25) (layer F.Cu) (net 17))
 (segment (start 146.7069 183.8512) (end 150.2035 183.8512) (width 0.25) (layer F.Cu) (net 17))
 (segment (start 150.2035 183.8512) (end 155.1147 178.94) (width 0.25) (layer F.Cu) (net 17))
 (segment (start 141 156.08) (end 141 157.2053) (width 0.25) (layer F.Cu) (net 18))
 (segment (start 145.7776 164.212) (end 142.5846 161.019) (width 0.25) (layer F.Cu) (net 18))
 (segment (start 142.5846 161.019) (end 142.5846 158.5086) (width 0.25) (layer F.Cu) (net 18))
 (segment (start 142.5846 158.5086) (end 141.2813 157.2053) (width 0.25) (layer F.Cu) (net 18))
 (segment (start 141.2813 157.2053) (end 141 157.2053) (width 0.25) (layer F.Cu) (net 18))
 (segment (start 145.1147 154.813) (end 145.1147 158.8143) (width 0.25) (layer F.Cu) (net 19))
 (segment (start 145.1147 158.8143) (end 146.5344 160.234) (width 0.25) (layer F.Cu) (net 19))
 (segment (start 146.3465 167.7595) (end 146.5627 167.5433) (width 0.25) (layer B.Cu) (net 19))
 (segment (start 146.5627 167.5433) (end 146.5627 160.2623) (width 0.25) (layer B.Cu) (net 19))
 (segment (start 146.5627 160.2623) (end 146.5344 160.234) (width 0.25) (layer B.Cu) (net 19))
 (segment (start 146.64 154.813) (end 145.1147 154.813) (width 0.25) (layer F.Cu) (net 19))
 (segment (start 146.3465 167.7595) (end 146.3465 172.7118) (width 0.25) (layer B.Cu) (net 19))
 (segment (start 146.3465 172.7118) (end 155.1147 181.48) (width 0.25) (layer B.Cu) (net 19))
 (segment (start 146.1392 167.7595) (end 146.3465 167.7595) (width 0.25) (layer B.Cu) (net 19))
 (segment (start 143.5149 168.5253) (end 144.3106 167.7296) (width 0.25) (layer F.Cu) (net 19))
 (segment (start 144.3106 167.7296) (end 144.3404 167.7595) (width 0.25) (layer F.Cu) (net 19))
 (segment (start 144.3404 167.7595) (end 146.1392 167.7595) (width 0.25) (layer F.Cu) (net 19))
 (segment (start 156.24 181.48) (end 155.1147 181.48) (width 0.25) (layer B.Cu) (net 19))
 (via (at 146.5344 160.234) (size 0.8) (layers F.Cu B.Cu) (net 19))
 (via (at 146.1392 167.7595) (size 0.8) (layers F.Cu B.Cu) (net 19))
 (segment (start 141 153.54) (end 141 154.6653) (width 0.25) (layer F.Cu) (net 20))
 (segment (start 146.3433 163.6463) (end 143.2087 160.5117) (width 0.25) (layer F.Cu) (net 20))
 (segment (start 143.2087 160.5117) (end 143.2087 156.5927) (width 0.25) (layer F.Cu) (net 20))
 (segment (start 143.2087 156.5927) (end 141.2813 154.6653) (width 0.25) (layer F.Cu) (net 20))
 (segment (start 141.2813 154.6653) (end 141 154.6653) (width 0.25) (layer F.Cu) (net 20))
 (segment (start 146.909 163.0806) (end 143.7638 159.9354) (width 0.25) (layer F.Cu) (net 22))
 (segment (start 143.7638 159.9354) (end 143.7638 154.6078) (width 0.25) (layer F.Cu) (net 22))
 (segment (start 143.7638 154.6078) (end 141.2813 152.1253) (width 0.25) (layer F.Cu) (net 22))
 (segment (start 141.2813 152.1253) (end 141 152.1253) (width 0.25) (layer F.Cu) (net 22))
 (segment (start 141 151) (end 141 152.1253) (width 0.25) (layer F.Cu) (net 22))
 (segment (start 152.9194 169.091) (end 153.7152 169.8868) (width 0.25) (layer F.Cu) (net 23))
 (segment (start 149.336 182.88) (end 150.1613 182.88) (width 0.25) (layer F.Cu) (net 23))
 (segment (start 150.1613 182.88) (end 153.7152 179.3261) (width 0.25) (layer F.Cu) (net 23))
 (segment (start 153.7152 179.3261) (end 153.7152 169.8868) (width 0.25) (layer F.Cu) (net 23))
 (segment (start 152.3537 169.6567) (end 153.1494 170.4524) (width 0.25) (layer F.Cu) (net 24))
 (segment (start 147.336 182.88) (end 148.1613 182.88) (width 0.25) (layer F.Cu) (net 24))
 (segment (start 148.1613 182.88) (end 148.1613 182.0547) (width 0.25) (layer F.Cu) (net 24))
 (segment (start 148.1613 182.0547) (end 153.1494 177.0666) (width 0.25) (layer F.Cu) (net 24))
 (segment (start 153.1494 177.0666) (end 153.1494 170.4524) (width 0.25) (layer F.Cu) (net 24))
 (segment (start 146.64 156.083) (end 146.64 158.9168) (width 0.25) (layer F.Cu) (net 25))
 (segment (start 146.64 158.9168) (end 147.2598 159.5366) (width 0.25) (layer F.Cu) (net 25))
 (segment (start 151.33 167.4603) (end 151.1717 167.4603) (width 0.25) (layer B.Cu) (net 25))
 (segment (start 151.1717 167.4603) (end 147.2598 163.5484) (width 0.25) (layer B.Cu) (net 25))
 (segment (start 147.2598 163.5484) (end 147.2598 159.5366) (width 0.25) (layer B.Cu) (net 25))
 (segment (start 151.788 170.2224) (end 152.5837 171.0181) (width 0.25) (layer F.Cu) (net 25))
 (segment (start 149.34 176.276) (end 149.9153 176.276) (width 0.25) (layer F.Cu) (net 25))
 (segment (start 149.9153 176.276) (end 152.5837 173.6076) (width 0.25) (layer F.Cu) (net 25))
 (segment (start 152.5837 173.6076) (end 152.5837 171.0181) (width 0.25) (layer F.Cu) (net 25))
 (segment (start 151.33 167.4603) (end 151.33 168.9151) (width 0.25) (layer F.Cu) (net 25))
 (segment (start 151.33 168.9151) (end 151.2591 168.986) (width 0.25) (layer F.Cu) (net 25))
 (segment (start 151.2591 168.986) (end 151.2591 169.6935) (width 0.25) (layer F.Cu) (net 25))
 (segment (start 151.2591 169.6935) (end 151.788 170.2224) (width 0.25) (layer F.Cu) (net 25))
 (via (at 151.33 167.4603) (size 0.8) (layers F.Cu B.Cu) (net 25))
 (via (at 147.2598 159.5366) (size 0.8) (layers F.Cu B.Cu) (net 25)))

